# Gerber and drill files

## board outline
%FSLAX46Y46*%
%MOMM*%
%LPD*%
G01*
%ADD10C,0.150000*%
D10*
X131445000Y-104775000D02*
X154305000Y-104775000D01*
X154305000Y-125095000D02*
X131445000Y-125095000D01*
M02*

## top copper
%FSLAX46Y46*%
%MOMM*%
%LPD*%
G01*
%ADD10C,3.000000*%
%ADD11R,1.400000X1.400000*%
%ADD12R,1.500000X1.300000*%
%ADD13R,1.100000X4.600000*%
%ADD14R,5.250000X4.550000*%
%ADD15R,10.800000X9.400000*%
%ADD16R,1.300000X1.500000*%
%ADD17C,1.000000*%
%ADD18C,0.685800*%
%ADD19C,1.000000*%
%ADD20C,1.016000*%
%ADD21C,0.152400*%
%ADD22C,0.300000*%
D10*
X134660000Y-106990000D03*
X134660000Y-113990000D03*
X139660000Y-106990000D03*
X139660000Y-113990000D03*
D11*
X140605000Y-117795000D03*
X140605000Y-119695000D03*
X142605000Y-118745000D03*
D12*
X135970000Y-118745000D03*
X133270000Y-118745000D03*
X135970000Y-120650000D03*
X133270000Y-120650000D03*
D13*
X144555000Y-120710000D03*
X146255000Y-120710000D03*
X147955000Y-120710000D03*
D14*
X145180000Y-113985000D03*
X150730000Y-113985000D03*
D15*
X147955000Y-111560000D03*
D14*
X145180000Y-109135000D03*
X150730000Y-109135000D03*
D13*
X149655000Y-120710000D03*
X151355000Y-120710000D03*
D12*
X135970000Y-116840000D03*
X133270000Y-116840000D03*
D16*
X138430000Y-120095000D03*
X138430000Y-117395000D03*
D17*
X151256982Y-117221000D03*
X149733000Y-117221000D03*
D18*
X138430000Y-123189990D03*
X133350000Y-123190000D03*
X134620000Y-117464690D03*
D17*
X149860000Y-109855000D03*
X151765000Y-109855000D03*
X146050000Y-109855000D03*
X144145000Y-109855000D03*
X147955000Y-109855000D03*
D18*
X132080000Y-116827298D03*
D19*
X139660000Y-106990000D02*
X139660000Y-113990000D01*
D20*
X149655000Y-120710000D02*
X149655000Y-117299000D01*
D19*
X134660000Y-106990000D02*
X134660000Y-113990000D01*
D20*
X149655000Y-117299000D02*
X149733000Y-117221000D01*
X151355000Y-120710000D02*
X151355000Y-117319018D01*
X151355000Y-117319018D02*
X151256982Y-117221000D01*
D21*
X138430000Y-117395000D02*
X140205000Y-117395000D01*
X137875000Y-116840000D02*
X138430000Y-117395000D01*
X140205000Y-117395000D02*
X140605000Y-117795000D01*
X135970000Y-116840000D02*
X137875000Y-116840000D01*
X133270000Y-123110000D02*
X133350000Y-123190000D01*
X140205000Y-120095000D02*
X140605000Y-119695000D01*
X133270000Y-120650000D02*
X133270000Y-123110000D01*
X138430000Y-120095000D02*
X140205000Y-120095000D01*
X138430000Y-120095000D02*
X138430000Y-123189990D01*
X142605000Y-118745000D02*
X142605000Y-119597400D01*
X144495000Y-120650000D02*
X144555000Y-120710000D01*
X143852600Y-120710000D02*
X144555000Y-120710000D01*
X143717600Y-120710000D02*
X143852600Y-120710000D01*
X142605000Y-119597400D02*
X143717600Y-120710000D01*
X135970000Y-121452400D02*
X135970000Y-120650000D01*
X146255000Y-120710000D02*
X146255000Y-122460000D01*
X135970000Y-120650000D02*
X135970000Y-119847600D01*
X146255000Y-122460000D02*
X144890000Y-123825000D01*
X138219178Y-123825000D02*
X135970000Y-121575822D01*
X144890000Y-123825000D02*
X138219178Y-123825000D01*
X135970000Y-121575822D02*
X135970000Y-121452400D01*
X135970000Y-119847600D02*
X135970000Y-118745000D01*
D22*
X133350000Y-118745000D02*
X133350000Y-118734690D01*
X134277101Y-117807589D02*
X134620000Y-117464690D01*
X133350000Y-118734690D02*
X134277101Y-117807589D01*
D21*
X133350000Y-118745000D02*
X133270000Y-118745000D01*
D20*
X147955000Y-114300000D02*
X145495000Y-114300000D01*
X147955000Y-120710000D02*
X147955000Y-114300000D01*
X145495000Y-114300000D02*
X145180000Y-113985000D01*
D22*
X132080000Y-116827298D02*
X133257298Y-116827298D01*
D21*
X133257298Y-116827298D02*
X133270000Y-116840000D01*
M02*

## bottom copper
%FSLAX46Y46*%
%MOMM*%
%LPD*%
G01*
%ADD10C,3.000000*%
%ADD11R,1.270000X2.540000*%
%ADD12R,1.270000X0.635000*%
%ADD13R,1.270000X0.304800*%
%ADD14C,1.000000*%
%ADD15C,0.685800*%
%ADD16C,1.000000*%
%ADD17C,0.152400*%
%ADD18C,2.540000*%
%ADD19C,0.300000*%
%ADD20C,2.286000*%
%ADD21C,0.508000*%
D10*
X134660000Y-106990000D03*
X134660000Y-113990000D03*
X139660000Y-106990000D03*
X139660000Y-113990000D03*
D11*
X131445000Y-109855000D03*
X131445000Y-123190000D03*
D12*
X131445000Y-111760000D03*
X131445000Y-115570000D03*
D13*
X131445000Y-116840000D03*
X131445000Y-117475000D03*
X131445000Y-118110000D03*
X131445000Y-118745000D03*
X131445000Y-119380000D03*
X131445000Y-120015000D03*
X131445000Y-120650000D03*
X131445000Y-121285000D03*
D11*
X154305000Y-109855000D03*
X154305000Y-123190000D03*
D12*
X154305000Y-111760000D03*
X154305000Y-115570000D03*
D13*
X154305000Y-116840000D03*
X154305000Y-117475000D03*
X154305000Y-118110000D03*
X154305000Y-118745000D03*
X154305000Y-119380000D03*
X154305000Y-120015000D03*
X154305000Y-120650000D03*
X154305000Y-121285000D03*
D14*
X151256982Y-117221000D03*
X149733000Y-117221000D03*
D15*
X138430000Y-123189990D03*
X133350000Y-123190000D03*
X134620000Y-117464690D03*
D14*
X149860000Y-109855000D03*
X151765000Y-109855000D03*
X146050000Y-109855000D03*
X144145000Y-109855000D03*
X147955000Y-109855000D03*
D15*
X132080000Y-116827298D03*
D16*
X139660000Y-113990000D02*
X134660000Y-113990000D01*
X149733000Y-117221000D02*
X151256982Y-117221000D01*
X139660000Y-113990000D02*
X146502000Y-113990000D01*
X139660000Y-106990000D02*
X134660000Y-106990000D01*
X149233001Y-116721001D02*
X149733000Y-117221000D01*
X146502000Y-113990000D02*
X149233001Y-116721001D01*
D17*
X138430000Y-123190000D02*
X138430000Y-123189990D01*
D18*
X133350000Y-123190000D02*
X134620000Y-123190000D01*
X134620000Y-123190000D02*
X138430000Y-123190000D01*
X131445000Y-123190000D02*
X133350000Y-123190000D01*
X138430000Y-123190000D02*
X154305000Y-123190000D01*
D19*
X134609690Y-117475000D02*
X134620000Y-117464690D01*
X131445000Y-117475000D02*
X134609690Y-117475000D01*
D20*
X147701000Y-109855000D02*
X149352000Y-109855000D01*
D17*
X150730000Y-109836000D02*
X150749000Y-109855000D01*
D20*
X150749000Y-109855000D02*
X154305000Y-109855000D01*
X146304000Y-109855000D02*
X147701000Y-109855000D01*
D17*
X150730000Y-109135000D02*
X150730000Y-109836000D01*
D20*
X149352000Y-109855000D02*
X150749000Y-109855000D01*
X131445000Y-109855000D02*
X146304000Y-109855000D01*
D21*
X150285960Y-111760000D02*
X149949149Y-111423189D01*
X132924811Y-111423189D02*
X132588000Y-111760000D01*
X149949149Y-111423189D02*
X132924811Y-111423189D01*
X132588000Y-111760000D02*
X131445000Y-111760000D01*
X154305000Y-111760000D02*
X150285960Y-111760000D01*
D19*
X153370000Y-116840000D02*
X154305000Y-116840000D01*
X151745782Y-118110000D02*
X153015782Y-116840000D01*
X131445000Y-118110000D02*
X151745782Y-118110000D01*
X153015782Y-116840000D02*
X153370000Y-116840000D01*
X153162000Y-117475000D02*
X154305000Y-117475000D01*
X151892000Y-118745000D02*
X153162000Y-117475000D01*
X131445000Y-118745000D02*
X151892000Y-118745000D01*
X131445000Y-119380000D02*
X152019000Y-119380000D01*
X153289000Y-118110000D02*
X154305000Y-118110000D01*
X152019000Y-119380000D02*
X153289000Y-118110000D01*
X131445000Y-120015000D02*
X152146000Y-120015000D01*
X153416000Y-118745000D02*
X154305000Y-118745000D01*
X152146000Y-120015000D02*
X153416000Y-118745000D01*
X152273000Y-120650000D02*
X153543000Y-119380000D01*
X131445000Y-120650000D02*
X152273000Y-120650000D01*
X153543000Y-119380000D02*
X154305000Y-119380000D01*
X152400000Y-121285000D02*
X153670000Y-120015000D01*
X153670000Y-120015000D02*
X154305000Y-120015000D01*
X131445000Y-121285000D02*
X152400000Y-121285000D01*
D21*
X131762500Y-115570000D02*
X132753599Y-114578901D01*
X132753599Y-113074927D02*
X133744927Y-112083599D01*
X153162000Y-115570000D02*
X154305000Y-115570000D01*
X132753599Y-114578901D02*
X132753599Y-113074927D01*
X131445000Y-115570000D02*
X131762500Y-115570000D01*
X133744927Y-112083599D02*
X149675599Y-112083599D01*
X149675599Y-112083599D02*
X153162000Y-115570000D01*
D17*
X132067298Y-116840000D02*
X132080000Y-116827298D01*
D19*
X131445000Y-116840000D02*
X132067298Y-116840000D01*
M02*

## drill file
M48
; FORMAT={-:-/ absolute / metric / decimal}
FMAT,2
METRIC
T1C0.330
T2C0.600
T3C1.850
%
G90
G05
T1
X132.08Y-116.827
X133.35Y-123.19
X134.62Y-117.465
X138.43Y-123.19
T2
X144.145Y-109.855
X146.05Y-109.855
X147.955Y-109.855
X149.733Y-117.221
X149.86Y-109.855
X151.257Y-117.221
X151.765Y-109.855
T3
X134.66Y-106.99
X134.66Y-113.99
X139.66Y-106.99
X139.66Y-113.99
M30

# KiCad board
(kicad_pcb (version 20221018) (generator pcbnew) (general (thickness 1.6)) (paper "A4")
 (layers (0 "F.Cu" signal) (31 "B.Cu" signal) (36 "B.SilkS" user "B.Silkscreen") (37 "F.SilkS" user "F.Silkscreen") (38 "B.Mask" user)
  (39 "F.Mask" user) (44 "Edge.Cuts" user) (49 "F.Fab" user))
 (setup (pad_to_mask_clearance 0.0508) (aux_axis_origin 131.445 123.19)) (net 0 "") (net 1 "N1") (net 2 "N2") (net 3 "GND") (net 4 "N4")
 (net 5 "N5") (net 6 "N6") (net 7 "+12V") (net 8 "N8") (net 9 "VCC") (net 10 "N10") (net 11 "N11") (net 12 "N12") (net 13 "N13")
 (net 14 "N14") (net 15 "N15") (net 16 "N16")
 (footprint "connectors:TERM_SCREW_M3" (layer "F.Cu") (at 137.16 110.49)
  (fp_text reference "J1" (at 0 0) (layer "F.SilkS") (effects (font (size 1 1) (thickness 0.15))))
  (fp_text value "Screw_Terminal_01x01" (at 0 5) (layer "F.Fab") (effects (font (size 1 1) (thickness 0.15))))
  (pad "1" thru_hole circle (at -2.5 -3.5) (size 3 3) (drill 1.85) (layers "*.Cu" "*.Mask") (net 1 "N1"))
  (pad "1" thru_hole circle (at -2.5 3.5) (size 3 3) (drill 1.85) (layers "*.Cu" "*.Mask") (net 1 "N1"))
  (pad "1" thru_hole circle (at 2.5 -3.5) (size 3 3) (drill 1.85) (layers "*.Cu" "*.Mask") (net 1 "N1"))
  (pad "1" thru_hole circle (at 2.5 3.5) (size 3 3) (drill 1.85) (layers "*.Cu" "*.Mask") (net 1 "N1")))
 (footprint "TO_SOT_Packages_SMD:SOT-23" (layer "F.Cu") (at 141.605 118.745)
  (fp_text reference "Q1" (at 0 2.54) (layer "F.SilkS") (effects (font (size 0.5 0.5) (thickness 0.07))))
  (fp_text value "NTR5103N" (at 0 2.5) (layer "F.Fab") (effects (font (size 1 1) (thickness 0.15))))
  (pad "1" smd rect (at -1 -0.95) (size 1.4 1.4) (layers "F.Cu" "F.Mask") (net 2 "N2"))
  (pad "2" smd rect (at -1 0.95) (size 1.4 1.4) (layers "F.Cu" "F.Mask") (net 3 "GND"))
  (pad "3" smd rect (at 1 0) (size 1.4 1.4) (layers "F.Cu" "F.Mask") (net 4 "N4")))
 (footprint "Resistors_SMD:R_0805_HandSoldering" (layer "F.Cu") (at 134.62 118.745 180)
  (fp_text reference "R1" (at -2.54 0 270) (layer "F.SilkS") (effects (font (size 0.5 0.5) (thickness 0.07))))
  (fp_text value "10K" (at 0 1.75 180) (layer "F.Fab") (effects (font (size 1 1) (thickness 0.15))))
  (pad "1" smd rect (at -1.35 0 180) (size 1.5 1.3) (layers "F.Cu" "F.Mask") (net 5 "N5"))
  (pad "2" smd rect (at 1.35 0 180) (size 1.5 1.3) (layers "F.Cu" "F.Mask") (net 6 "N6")))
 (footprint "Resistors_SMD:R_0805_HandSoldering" (layer "F.Cu") (at 134.62 120.65 180)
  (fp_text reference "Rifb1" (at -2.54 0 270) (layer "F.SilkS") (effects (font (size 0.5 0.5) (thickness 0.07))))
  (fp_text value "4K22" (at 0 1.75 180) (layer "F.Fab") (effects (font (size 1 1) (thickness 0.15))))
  (pad "1" smd rect (at -1.35 0 180) (size 1.5 1.3) (layers "F.Cu" "F.Mask") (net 5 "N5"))
  (pad "2" smd rect (at 1.35 0 180) (size 1.5 1.3) (layers "F.Cu" "F.Mask") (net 3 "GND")))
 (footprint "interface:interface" (layer "F.Cu") (at 131.445 105.41)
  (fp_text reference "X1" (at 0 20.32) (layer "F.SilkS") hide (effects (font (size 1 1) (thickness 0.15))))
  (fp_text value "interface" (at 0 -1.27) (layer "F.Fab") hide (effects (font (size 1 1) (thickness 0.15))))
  (pad "1" smd rect (at 0 4.445) (size 1.27 2.54) (layers "B.Cu") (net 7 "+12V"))
  (pad "2" smd rect (at 0 17.78) (size 1.27 2.54) (layers "B.Cu") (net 3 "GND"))
  (pad "3" smd rect (at 0 6.35) (size 1.27 0.635) (layers "B.Cu") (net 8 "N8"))
  (pad "4" smd rect (at 0 10.16) (size 1.27 0.635) (layers "B.Cu") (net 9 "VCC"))
  (pad "5" smd rect (at 0 11.43) (size 1.27 0.3048) (layers "B.Cu") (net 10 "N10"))
  (pad "6" smd rect (at 0 12.065) (size 1.27 0.3048) (layers "B.Cu") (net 6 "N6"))
  (pad "7" smd rect (at 0 12.7) (size 1.27 0.3048) (layers "B.Cu") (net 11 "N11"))
  (pad "8" smd rect (at 0 13.335) (size 1.27 0.3048) (layers "B.Cu") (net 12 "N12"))
  (pad "9" smd rect (at 0 13.97) (size 1.27 0.3048) (layers "B.Cu") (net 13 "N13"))
  (pad "10" smd rect (at 0 14.605) (size 1.27 0.3048) (layers "B.Cu") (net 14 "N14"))
  (pad "11" smd rect (at 0 15.24) (size 1.27 0.3048) (layers "B.Cu") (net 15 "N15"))
  (pad "12" smd rect (at 0 15.875) (size 1.27 0.3048) (layers "B.Cu") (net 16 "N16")))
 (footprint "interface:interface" (layer "F.Cu") (at 154.305 105.41)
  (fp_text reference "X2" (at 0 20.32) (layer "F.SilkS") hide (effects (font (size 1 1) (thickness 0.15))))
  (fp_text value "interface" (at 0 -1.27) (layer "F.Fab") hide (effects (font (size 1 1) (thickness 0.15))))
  (pad "1" smd rect (at 0 4.445) (size 1.27 2.54) (layers "B.Cu") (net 7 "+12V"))
  (pad "2" smd rect (at 0 17.78) (size 1.27 2.54) (layers "B.Cu") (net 3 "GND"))
  (pad "3" smd rect (at 0 6.35) (size 1.27 0.635) (layers "B.Cu") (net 8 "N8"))
  (pad "4" smd rect (at 0 10.16) (size 1.27 0.635) (layers "B.Cu") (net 9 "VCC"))
  (pad "5" smd rect (at 0 11.43) (size 1.27 0.3048) (layers "B.Cu") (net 11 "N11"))
  (pad "6" smd rect (at 0 12.065) (size 1.27 0.3048) (layers "B.Cu") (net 12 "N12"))
  (pad "7" smd rect (at 0 12.7) (size 1.27 0.3048) (layers "B.Cu") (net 13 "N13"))
  (pad "8" smd rect (at 0 13.335) (size 1.27 0.3048) (layers "B.Cu") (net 14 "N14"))
  (pad "9" smd rect (at 0 13.97) (size 1.27 0.3048) (layers "B.Cu") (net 15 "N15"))
  (pad "10" smd rect (at 0 14.605) (size 1.27 0.3048) (layers "B.Cu") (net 16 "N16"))
  (pad "11" smd rect (at 0 15.24) (size 1.27 0.3048) (layers "B.Cu"))
  (pad "12" smd rect (at 0 15.875) (size 1.27 0.3048) (layers "B.Cu")))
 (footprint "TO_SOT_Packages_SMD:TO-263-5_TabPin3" (layer "F.Cu") (at 147.955 114.935 90)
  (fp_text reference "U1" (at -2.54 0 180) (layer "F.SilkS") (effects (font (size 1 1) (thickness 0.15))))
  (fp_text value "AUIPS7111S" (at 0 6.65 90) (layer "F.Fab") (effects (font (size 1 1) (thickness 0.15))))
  (pad "1" smd rect (at -5.775 -3.4 90) (size 4.6 1.1) (layers "F.Cu" "F.Mask") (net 4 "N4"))
  (pad "2" smd rect (at -5.775 -1.7 90) (size 4.6 1.1) (layers "F.Cu" "F.Mask") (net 5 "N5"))
  (pad "3" smd rect (at -5.775 0 90) (size 4.6 1.1) (layers "F.Cu" "F.Mask") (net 7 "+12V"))
  (pad "3" smd rect (at 0.95 -2.775 90) (size 4.55 5.25) (layers "F.Cu") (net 7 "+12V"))
  (pad "3" smd rect (at 0.95 2.775 90) (size 4.55 5.25) (layers "F.Cu") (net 7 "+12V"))
  (pad "3" smd rect (at 3.375 0 90) (size 9.4 10.8) (layers "F.Cu" "F.Mask") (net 7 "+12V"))
  (pad "3" smd rect (at 5.8 -2.775 90) (size 4.55 5.25) (layers "F.Cu") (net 7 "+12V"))
  (pad "3" smd rect (at 5.8 2.775 90) (size 4.55 5.25) (layers "F.Cu") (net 7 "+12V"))
  (pad "4" smd rect (at -5.775 1.7 90) (size 4.6 1.1) (layers "F.Cu" "F.Mask") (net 1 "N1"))
  (pad "5" smd rect (at -5.775 3.4 90) (size 4.6 1.1) (layers "F.Cu" "F.Mask") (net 1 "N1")))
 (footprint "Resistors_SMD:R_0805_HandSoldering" (layer "F.Cu") (at 134.62 116.84 180)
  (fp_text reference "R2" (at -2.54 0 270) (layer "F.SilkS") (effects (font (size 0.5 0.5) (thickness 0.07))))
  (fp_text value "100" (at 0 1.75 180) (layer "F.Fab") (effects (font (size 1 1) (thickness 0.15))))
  (pad "1" smd rect (at -1.35 0 180) (size 1.5 1.3) (layers "F.Cu" "F.Mask") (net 2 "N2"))
  (pad "2" smd rect (at 1.35 0 180) (size 1.5 1.3) (layers "F.Cu" "F.Mask") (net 10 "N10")))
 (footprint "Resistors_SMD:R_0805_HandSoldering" (layer "F.Cu") (at 138.43 118.745 90)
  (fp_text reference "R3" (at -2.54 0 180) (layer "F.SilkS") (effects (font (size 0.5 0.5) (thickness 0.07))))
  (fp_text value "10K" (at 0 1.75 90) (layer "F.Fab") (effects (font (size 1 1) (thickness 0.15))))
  (pad "1" smd rect (at -1.35 0 90) (size 1.5 1.3) (layers "F.Cu" "F.Mask") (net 3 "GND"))
  (pad "2" smd rect (at 1.35 0 90) (size 1.5 1.3) (layers "F.Cu" "F.Mask") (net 2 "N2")))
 (gr_line (start 131.445 104.775) (end 154.305 104.775) (stroke (width 0.15) (type solid)) (layer "Edge.Cuts"))
 (gr_line (start 154.305 125.095) (end 131.445 125.095) (stroke (width 0.15) (type solid)) (layer "Edge.Cuts"))
 (segment (start 139.66 106.99) (end 139.66 113.99) (width 1) (layer "F.Cu") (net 1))
 (segment (start 149.655 120.71) (end 149.655 117.299) (width 1.016) (layer "F.Cu") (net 1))
 (segment (start 134.66 106.99) (end 134.66 113.99) (width 1) (layer "F.Cu") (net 1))
 (segment (start 149.655 117.299) (end 149.733 117.221) (width 1.016) (layer "F.Cu") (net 1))
 (segment (start 151.355 120.71) (end 151.355 117.319018) (width 1.016) (layer "F.Cu") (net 1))
 (segment (start 151.355 117.319018) (end 151.256982 117.221) (width 1.016) (layer "F.Cu") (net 1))
 (via (at 151.256982 117.221) (size 1) (drill 0.6) (layers "F.Cu" "B.Cu") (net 1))
 (via (at 149.733 117.221) (size 1) (drill 0.6) (layers "F.Cu" "B.Cu") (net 1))
 (segment (start 139.66 113.99) (end 134.66 113.99) (width 1) (layer "B.Cu") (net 1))
 (segment (start 149.733 117.221) (end 151.256982 117.221) (width 1) (layer "B.Cu") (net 1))
 (segment (start 139.66 113.99) (end 146.502 113.99) (width 1) (layer "B.Cu") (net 1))
 (segment (start 139.66 106.99) (end 134.66 106.99) (width 1) (layer "B.Cu") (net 1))
 (segment (start 149.233001 116.721001) (end 149.733 117.221) (width 1) (layer "B.Cu") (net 1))
 (segment (start 146.502 113.99) (end 149.233001 116.721001) (width 1) (layer "B.Cu") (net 1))
 (segment (start 138.43 117.395) (end 140.205 117.395) (width 0.1524) (layer "F.Cu") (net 2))
 (segment (start 137.875 116.84) (end 138.43 117.395) (width 0.1524) (layer "F.Cu") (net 2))
 (segment (start 140.205 117.395) (end 140.605 117.795) (width 0.1524) (layer "F.Cu") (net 2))
 (segment (start 135.97 116.84) (end 137.875 116.84) (width 0.1524) (layer "F.Cu") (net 2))
 (segment (start 133.27 123.11) (end 133.35 123.19) (width 0.1524) (layer "F.Cu") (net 3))
 (segment (start 140.205 120.095) (end 140.605 119.695) (width 0.1524) (layer "F.Cu") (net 3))
 (segment (start 133.27 120.65) (end 133.27 123.11) (width 0.1524) (layer "F.Cu") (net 3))
 (segment (start 138.43 120.095) (end 140.205 120.095) (width 0.1524) (layer "F.Cu") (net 3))
 (segment (start 138.43 120.095) (end 138.43 123.18999) (width 0.1524) (layer "F.Cu") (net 3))
 (via (at 138.43 123.18999) (size 0.6858) (drill 0.3302) (layers "F.Cu" "B.Cu") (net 3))
 (via (at 133.35 123.19) (size 0.6858) (drill 0.3302) (layers "F.Cu" "B.Cu") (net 3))
 (segment (start 138.43 123.19) (end 138.43 123.18999) (width 0.1524) (layer "B.Cu") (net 3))
 (segment (start 133.35 123.19) (end 134.62 123.19) (width 2.54) (layer "B.Cu") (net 3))
 (segment (start 134.62 123.19) (end 138.43 123.19) (width 2.54) (layer "B.Cu") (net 3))
 (segment (start 131.445 123.19) (end 133.35 123.19) (width 2.54) (layer "B.Cu") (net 3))
 (segment (start 138.43 123.19) (end 154.305 123.19) (width 2.54) (layer "B.Cu") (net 3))
 (segment (start 142.605 118.745) (end 142.605 119.5974) (width 0.1524) (layer "F.Cu") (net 4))
 (segment (start 144.495 120.65) (end 144.555 120.71) (width 0.1524) (layer "F.Cu") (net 4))
 (segment (start 143.8526 120.71) (end 144.555 120.71) (width 0.1524) (layer "F.Cu") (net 4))
 (segment (start 143.7176 120.71) (end 143.8526 120.71) (width 0.1524) (layer "F.Cu") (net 4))
 (segment (start 142.605 119.5974) (end 143.7176 120.71) (width 0.1524) (layer "F.Cu") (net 4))
 (segment (start 135.97 121.4524) (end 135.97 120.65) (width 0.1524) (layer "F.Cu") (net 5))
 (segment (start 146.255 120.71) (end 146.255 122.46) (width 0.1524) (layer "F.Cu") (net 5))
 (segment (start 135.97 120.65) (end 135.97 119.8476) (width 0.1524) (layer "F.Cu") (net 5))
 (segment (start 146.255 122.46) (end 144.89 123.825) (width 0.1524) (layer "F.Cu") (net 5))
 (segment (start 138.219178 123.825) (end 135.97 121.575822) (width 0.1524) (layer "F.Cu") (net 5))
 (segment (start 144.89 123.825) (end 138.219178 123.825) (width 0.1524) (layer "F.Cu") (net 5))
 (segment (start 135.97 121.575822) (end 135.97 121.4524) (width 0.1524) (layer "F.Cu") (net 5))
 (segment (start 135.97 119.8476) (end 135.97 118.745) (width 0.1524) (layer "F.Cu") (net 5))
 (segment (start 133.35 118.745) (end 133.35 118.73469) (width 0.3) (layer "F.Cu") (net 6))
 (segment (start 134.277101 117.807589) (end 134.62 117.46469) (width 0.3) (layer "F.Cu") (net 6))
 (segment (start 133.35 118.73469) (end 134.277101 117.807589) (width 0.3) (layer "F.Cu") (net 6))
 (segment (start 133.35 118.745) (end 133.27 118.745) (width 0.1524) (layer "F.Cu") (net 6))
 (via (at 134.62 117.46469) (size 0.6858) (drill 0.3302) (layers "F.Cu" "B.Cu") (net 6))
 (segment (start 134.60969 117.475) (end 134.62 117.46469) (width 0.3) (layer "B.Cu") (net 6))
 (segment (start 131.445 117.475) (end 134.60969 117.475) (width 0.3) (layer "B.Cu") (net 6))
 (segment (start 147.955 114.3) (end 145.495 114.3) (width 1.016) (layer "F.Cu") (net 7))
 (segment (start 147.955 120.71) (end 147.955 114.3) (width 1.016) (layer "F.Cu") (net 7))
 (segment (start 145.495 114.3) (end 145.18 113.985) (width 1.016) (layer "F.Cu") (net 7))
 (via (at 149.86 109.855) (size 1) (drill 0.6) (layers "F.Cu" "B.Cu") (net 7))
 (via (at 151.765 109.855) (size 1) (drill 0.6) (layers "F.Cu" "B.Cu") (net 7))
 (via (at 146.05 109.855) (size 1) (drill 0.6) (layers "F.Cu" "B.Cu") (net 7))
 (via (at 144.145 109.855) (size 1) (drill 0.6) (layers "F.Cu" "B.Cu") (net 7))
 (via (at 147.955 109.855) (size 1) (drill 0.6) (layers "F.Cu" "B.Cu") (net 7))
 (segment (start 147.701 109.855) (end 149.352 109.855) (width 2.286) (layer "B.Cu") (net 7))
 (segment (start 150.73 109.836) (end 150.749 109.855) (width 0.1524) (layer "B.Cu") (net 7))
 (segment (start 150.749 109.855) (end 154.305 109.855) (width 2.286) (layer "B.Cu") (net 7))
 (segment (start 146.304 109.855) (end 147.701 109.855) (width 2.286) (layer "B.Cu") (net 7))
 (segment (start 150.73 109.135) (end 150.73 109.836) (width 0.1524) (layer "B.Cu") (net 7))
 (segment (start 149.352 109.855) (end 150.749 109.855) (width 2.286) (layer "B.Cu") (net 7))
 (segment (start 131.445 109.855) (end 146.304 109.855) (width 2.286) (layer "B.Cu") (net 7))
 (segment (start 150.28596 111.76) (end 149.949149 111.423189) (width 0.508) (layer "B.Cu") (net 8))
 (segment (start 132.924811 111.423189) (end 132.588 111.76) (width 0.508) (layer "B.Cu") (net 8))
 (segment (start 149.949149 111.423189) (end 132.924811 111.423189) (width 0.508) (layer "B.Cu") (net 8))
 (segment (start 132.588 111.76) (end 131.445 111.76) (width 0.508) (layer "B.Cu") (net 8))
 (segment (start 154.305 111.76) (end 150.28596 111.76) (width 0.508) (layer "B.Cu") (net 8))
 (segment (start 153.37 116.84) (end 154.305 116.84) (width 0.3) (layer "B.Cu") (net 11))
 (segment (start 151.745782 118.11) (end 153.015782 116.84) (width 0.3) (layer "B.Cu") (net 11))
 (segment (start 131.445 118.11) (end 151.745782 118.11) (width 0.3) (layer "B.Cu") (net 11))
 (segment (start 153.015782 116.84) (end 153.37 116.84) (width 0.3) (layer "B.Cu") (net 11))
 (segment (start 153.162 117.475) (end 154.305 117.475) (width 0.3) (layer "B.Cu") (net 12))
 (segment (start 151.892 118.745) (end 153.162 117.475) (width 0.3) (layer "B.Cu") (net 12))
 (segment (start 131.445 118.745) (end 151.892 118.745) (width 0.3) (layer "B.Cu") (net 12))
 (segment (start 131.445 119.38) (end 152.019 119.38) (width 0.3) (layer "B.Cu") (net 13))
 (segment (start 153.289 118.11) (end 154.305 118.11) (width 0.3) (layer "B.Cu") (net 13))
 (segment (start 152.019 119.38) (end 153.289 118.11) (width 0.3) (layer "B.Cu") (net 13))
 (segment (start 131.445 120.015) (end 152.146 120.015) (width 0.3) (layer "B.Cu") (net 14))
 (segment (start 153.416 118.745) (end 154.305 118.745) (width 0.3) (layer "B.Cu") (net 14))
 (segment (start 152.146 120.015) (end 153.416 118.745) (width 0.3) (layer "B.Cu") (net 14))
 (segment (start 152.273 120.65) (end 153.543 119.38) (width 0.3) (layer "B.Cu") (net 15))
 (segment (start 131.445 120.65) (end 152.273 120.65) (width 0.3) (layer "B.Cu") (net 15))
 (segment (start 153.543 119.38) (end 154.305 119.38) (width 0.3) (layer "B.Cu") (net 15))
 (segment (start 152.4 121.285) (end 153.67 120.015) (width 0.3) (layer "B.Cu") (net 16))
 (segment (start 153.67 120.015) (end 154.305 120.015) (width 0.3) (layer "B.Cu") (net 16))
 (segment (start 131.445 121.285) (end 152.4 121.285) (width 0.3) (layer "B.Cu") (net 16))
 (segment (start 131.7625 115.57) (end 132.753599 114.578901) (width 0.508) (layer "B.Cu") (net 9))
 (segment (start 132.753599 113.074927) (end 133.744927 112.083599) (width 0.508) (layer "B.Cu") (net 9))
 (segment (start 153.162 115.57) (end 154.305 115.57) (width 0.508) (layer "B.Cu") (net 9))
 (segment (start 132.753599 114.578901) (end 132.753599 113.074927) (width 0.508) (layer "B.Cu") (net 9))
 (segment (start 131.445 115.57) (end 131.7625 115.57) (width 0.508) (layer "B.Cu") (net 9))
 (segment (start 133.744927 112.083599) (end 149.675599 112.083599) (width 0.508) (layer "B.Cu") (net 9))
 (segment (start 149.675599 112.083599) (end 153.162 115.57) (width 0.508) (layer "B.Cu") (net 9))
 (segment (start 132.08 116.827298) (end 133.257298 116.827298) (width 0.3) (layer "F.Cu") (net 10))
 (segment (start 133.257298 116.827298) (end 133.27 116.84) (width 0.1524) (layer "F.Cu") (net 10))
 (via (at 132.08 116.827298) (size 0.6858) (drill 0.3302) (layers "F.Cu" "B.Cu") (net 10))
 (segment (start 132.067298 116.84) (end 132.08 116.827298) (width 0.1524) (layer "B.Cu") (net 10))
 (segment (start 131.445 116.84) (end 132.067298 116.84) (width 0.3) (layer "B.Cu") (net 10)))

